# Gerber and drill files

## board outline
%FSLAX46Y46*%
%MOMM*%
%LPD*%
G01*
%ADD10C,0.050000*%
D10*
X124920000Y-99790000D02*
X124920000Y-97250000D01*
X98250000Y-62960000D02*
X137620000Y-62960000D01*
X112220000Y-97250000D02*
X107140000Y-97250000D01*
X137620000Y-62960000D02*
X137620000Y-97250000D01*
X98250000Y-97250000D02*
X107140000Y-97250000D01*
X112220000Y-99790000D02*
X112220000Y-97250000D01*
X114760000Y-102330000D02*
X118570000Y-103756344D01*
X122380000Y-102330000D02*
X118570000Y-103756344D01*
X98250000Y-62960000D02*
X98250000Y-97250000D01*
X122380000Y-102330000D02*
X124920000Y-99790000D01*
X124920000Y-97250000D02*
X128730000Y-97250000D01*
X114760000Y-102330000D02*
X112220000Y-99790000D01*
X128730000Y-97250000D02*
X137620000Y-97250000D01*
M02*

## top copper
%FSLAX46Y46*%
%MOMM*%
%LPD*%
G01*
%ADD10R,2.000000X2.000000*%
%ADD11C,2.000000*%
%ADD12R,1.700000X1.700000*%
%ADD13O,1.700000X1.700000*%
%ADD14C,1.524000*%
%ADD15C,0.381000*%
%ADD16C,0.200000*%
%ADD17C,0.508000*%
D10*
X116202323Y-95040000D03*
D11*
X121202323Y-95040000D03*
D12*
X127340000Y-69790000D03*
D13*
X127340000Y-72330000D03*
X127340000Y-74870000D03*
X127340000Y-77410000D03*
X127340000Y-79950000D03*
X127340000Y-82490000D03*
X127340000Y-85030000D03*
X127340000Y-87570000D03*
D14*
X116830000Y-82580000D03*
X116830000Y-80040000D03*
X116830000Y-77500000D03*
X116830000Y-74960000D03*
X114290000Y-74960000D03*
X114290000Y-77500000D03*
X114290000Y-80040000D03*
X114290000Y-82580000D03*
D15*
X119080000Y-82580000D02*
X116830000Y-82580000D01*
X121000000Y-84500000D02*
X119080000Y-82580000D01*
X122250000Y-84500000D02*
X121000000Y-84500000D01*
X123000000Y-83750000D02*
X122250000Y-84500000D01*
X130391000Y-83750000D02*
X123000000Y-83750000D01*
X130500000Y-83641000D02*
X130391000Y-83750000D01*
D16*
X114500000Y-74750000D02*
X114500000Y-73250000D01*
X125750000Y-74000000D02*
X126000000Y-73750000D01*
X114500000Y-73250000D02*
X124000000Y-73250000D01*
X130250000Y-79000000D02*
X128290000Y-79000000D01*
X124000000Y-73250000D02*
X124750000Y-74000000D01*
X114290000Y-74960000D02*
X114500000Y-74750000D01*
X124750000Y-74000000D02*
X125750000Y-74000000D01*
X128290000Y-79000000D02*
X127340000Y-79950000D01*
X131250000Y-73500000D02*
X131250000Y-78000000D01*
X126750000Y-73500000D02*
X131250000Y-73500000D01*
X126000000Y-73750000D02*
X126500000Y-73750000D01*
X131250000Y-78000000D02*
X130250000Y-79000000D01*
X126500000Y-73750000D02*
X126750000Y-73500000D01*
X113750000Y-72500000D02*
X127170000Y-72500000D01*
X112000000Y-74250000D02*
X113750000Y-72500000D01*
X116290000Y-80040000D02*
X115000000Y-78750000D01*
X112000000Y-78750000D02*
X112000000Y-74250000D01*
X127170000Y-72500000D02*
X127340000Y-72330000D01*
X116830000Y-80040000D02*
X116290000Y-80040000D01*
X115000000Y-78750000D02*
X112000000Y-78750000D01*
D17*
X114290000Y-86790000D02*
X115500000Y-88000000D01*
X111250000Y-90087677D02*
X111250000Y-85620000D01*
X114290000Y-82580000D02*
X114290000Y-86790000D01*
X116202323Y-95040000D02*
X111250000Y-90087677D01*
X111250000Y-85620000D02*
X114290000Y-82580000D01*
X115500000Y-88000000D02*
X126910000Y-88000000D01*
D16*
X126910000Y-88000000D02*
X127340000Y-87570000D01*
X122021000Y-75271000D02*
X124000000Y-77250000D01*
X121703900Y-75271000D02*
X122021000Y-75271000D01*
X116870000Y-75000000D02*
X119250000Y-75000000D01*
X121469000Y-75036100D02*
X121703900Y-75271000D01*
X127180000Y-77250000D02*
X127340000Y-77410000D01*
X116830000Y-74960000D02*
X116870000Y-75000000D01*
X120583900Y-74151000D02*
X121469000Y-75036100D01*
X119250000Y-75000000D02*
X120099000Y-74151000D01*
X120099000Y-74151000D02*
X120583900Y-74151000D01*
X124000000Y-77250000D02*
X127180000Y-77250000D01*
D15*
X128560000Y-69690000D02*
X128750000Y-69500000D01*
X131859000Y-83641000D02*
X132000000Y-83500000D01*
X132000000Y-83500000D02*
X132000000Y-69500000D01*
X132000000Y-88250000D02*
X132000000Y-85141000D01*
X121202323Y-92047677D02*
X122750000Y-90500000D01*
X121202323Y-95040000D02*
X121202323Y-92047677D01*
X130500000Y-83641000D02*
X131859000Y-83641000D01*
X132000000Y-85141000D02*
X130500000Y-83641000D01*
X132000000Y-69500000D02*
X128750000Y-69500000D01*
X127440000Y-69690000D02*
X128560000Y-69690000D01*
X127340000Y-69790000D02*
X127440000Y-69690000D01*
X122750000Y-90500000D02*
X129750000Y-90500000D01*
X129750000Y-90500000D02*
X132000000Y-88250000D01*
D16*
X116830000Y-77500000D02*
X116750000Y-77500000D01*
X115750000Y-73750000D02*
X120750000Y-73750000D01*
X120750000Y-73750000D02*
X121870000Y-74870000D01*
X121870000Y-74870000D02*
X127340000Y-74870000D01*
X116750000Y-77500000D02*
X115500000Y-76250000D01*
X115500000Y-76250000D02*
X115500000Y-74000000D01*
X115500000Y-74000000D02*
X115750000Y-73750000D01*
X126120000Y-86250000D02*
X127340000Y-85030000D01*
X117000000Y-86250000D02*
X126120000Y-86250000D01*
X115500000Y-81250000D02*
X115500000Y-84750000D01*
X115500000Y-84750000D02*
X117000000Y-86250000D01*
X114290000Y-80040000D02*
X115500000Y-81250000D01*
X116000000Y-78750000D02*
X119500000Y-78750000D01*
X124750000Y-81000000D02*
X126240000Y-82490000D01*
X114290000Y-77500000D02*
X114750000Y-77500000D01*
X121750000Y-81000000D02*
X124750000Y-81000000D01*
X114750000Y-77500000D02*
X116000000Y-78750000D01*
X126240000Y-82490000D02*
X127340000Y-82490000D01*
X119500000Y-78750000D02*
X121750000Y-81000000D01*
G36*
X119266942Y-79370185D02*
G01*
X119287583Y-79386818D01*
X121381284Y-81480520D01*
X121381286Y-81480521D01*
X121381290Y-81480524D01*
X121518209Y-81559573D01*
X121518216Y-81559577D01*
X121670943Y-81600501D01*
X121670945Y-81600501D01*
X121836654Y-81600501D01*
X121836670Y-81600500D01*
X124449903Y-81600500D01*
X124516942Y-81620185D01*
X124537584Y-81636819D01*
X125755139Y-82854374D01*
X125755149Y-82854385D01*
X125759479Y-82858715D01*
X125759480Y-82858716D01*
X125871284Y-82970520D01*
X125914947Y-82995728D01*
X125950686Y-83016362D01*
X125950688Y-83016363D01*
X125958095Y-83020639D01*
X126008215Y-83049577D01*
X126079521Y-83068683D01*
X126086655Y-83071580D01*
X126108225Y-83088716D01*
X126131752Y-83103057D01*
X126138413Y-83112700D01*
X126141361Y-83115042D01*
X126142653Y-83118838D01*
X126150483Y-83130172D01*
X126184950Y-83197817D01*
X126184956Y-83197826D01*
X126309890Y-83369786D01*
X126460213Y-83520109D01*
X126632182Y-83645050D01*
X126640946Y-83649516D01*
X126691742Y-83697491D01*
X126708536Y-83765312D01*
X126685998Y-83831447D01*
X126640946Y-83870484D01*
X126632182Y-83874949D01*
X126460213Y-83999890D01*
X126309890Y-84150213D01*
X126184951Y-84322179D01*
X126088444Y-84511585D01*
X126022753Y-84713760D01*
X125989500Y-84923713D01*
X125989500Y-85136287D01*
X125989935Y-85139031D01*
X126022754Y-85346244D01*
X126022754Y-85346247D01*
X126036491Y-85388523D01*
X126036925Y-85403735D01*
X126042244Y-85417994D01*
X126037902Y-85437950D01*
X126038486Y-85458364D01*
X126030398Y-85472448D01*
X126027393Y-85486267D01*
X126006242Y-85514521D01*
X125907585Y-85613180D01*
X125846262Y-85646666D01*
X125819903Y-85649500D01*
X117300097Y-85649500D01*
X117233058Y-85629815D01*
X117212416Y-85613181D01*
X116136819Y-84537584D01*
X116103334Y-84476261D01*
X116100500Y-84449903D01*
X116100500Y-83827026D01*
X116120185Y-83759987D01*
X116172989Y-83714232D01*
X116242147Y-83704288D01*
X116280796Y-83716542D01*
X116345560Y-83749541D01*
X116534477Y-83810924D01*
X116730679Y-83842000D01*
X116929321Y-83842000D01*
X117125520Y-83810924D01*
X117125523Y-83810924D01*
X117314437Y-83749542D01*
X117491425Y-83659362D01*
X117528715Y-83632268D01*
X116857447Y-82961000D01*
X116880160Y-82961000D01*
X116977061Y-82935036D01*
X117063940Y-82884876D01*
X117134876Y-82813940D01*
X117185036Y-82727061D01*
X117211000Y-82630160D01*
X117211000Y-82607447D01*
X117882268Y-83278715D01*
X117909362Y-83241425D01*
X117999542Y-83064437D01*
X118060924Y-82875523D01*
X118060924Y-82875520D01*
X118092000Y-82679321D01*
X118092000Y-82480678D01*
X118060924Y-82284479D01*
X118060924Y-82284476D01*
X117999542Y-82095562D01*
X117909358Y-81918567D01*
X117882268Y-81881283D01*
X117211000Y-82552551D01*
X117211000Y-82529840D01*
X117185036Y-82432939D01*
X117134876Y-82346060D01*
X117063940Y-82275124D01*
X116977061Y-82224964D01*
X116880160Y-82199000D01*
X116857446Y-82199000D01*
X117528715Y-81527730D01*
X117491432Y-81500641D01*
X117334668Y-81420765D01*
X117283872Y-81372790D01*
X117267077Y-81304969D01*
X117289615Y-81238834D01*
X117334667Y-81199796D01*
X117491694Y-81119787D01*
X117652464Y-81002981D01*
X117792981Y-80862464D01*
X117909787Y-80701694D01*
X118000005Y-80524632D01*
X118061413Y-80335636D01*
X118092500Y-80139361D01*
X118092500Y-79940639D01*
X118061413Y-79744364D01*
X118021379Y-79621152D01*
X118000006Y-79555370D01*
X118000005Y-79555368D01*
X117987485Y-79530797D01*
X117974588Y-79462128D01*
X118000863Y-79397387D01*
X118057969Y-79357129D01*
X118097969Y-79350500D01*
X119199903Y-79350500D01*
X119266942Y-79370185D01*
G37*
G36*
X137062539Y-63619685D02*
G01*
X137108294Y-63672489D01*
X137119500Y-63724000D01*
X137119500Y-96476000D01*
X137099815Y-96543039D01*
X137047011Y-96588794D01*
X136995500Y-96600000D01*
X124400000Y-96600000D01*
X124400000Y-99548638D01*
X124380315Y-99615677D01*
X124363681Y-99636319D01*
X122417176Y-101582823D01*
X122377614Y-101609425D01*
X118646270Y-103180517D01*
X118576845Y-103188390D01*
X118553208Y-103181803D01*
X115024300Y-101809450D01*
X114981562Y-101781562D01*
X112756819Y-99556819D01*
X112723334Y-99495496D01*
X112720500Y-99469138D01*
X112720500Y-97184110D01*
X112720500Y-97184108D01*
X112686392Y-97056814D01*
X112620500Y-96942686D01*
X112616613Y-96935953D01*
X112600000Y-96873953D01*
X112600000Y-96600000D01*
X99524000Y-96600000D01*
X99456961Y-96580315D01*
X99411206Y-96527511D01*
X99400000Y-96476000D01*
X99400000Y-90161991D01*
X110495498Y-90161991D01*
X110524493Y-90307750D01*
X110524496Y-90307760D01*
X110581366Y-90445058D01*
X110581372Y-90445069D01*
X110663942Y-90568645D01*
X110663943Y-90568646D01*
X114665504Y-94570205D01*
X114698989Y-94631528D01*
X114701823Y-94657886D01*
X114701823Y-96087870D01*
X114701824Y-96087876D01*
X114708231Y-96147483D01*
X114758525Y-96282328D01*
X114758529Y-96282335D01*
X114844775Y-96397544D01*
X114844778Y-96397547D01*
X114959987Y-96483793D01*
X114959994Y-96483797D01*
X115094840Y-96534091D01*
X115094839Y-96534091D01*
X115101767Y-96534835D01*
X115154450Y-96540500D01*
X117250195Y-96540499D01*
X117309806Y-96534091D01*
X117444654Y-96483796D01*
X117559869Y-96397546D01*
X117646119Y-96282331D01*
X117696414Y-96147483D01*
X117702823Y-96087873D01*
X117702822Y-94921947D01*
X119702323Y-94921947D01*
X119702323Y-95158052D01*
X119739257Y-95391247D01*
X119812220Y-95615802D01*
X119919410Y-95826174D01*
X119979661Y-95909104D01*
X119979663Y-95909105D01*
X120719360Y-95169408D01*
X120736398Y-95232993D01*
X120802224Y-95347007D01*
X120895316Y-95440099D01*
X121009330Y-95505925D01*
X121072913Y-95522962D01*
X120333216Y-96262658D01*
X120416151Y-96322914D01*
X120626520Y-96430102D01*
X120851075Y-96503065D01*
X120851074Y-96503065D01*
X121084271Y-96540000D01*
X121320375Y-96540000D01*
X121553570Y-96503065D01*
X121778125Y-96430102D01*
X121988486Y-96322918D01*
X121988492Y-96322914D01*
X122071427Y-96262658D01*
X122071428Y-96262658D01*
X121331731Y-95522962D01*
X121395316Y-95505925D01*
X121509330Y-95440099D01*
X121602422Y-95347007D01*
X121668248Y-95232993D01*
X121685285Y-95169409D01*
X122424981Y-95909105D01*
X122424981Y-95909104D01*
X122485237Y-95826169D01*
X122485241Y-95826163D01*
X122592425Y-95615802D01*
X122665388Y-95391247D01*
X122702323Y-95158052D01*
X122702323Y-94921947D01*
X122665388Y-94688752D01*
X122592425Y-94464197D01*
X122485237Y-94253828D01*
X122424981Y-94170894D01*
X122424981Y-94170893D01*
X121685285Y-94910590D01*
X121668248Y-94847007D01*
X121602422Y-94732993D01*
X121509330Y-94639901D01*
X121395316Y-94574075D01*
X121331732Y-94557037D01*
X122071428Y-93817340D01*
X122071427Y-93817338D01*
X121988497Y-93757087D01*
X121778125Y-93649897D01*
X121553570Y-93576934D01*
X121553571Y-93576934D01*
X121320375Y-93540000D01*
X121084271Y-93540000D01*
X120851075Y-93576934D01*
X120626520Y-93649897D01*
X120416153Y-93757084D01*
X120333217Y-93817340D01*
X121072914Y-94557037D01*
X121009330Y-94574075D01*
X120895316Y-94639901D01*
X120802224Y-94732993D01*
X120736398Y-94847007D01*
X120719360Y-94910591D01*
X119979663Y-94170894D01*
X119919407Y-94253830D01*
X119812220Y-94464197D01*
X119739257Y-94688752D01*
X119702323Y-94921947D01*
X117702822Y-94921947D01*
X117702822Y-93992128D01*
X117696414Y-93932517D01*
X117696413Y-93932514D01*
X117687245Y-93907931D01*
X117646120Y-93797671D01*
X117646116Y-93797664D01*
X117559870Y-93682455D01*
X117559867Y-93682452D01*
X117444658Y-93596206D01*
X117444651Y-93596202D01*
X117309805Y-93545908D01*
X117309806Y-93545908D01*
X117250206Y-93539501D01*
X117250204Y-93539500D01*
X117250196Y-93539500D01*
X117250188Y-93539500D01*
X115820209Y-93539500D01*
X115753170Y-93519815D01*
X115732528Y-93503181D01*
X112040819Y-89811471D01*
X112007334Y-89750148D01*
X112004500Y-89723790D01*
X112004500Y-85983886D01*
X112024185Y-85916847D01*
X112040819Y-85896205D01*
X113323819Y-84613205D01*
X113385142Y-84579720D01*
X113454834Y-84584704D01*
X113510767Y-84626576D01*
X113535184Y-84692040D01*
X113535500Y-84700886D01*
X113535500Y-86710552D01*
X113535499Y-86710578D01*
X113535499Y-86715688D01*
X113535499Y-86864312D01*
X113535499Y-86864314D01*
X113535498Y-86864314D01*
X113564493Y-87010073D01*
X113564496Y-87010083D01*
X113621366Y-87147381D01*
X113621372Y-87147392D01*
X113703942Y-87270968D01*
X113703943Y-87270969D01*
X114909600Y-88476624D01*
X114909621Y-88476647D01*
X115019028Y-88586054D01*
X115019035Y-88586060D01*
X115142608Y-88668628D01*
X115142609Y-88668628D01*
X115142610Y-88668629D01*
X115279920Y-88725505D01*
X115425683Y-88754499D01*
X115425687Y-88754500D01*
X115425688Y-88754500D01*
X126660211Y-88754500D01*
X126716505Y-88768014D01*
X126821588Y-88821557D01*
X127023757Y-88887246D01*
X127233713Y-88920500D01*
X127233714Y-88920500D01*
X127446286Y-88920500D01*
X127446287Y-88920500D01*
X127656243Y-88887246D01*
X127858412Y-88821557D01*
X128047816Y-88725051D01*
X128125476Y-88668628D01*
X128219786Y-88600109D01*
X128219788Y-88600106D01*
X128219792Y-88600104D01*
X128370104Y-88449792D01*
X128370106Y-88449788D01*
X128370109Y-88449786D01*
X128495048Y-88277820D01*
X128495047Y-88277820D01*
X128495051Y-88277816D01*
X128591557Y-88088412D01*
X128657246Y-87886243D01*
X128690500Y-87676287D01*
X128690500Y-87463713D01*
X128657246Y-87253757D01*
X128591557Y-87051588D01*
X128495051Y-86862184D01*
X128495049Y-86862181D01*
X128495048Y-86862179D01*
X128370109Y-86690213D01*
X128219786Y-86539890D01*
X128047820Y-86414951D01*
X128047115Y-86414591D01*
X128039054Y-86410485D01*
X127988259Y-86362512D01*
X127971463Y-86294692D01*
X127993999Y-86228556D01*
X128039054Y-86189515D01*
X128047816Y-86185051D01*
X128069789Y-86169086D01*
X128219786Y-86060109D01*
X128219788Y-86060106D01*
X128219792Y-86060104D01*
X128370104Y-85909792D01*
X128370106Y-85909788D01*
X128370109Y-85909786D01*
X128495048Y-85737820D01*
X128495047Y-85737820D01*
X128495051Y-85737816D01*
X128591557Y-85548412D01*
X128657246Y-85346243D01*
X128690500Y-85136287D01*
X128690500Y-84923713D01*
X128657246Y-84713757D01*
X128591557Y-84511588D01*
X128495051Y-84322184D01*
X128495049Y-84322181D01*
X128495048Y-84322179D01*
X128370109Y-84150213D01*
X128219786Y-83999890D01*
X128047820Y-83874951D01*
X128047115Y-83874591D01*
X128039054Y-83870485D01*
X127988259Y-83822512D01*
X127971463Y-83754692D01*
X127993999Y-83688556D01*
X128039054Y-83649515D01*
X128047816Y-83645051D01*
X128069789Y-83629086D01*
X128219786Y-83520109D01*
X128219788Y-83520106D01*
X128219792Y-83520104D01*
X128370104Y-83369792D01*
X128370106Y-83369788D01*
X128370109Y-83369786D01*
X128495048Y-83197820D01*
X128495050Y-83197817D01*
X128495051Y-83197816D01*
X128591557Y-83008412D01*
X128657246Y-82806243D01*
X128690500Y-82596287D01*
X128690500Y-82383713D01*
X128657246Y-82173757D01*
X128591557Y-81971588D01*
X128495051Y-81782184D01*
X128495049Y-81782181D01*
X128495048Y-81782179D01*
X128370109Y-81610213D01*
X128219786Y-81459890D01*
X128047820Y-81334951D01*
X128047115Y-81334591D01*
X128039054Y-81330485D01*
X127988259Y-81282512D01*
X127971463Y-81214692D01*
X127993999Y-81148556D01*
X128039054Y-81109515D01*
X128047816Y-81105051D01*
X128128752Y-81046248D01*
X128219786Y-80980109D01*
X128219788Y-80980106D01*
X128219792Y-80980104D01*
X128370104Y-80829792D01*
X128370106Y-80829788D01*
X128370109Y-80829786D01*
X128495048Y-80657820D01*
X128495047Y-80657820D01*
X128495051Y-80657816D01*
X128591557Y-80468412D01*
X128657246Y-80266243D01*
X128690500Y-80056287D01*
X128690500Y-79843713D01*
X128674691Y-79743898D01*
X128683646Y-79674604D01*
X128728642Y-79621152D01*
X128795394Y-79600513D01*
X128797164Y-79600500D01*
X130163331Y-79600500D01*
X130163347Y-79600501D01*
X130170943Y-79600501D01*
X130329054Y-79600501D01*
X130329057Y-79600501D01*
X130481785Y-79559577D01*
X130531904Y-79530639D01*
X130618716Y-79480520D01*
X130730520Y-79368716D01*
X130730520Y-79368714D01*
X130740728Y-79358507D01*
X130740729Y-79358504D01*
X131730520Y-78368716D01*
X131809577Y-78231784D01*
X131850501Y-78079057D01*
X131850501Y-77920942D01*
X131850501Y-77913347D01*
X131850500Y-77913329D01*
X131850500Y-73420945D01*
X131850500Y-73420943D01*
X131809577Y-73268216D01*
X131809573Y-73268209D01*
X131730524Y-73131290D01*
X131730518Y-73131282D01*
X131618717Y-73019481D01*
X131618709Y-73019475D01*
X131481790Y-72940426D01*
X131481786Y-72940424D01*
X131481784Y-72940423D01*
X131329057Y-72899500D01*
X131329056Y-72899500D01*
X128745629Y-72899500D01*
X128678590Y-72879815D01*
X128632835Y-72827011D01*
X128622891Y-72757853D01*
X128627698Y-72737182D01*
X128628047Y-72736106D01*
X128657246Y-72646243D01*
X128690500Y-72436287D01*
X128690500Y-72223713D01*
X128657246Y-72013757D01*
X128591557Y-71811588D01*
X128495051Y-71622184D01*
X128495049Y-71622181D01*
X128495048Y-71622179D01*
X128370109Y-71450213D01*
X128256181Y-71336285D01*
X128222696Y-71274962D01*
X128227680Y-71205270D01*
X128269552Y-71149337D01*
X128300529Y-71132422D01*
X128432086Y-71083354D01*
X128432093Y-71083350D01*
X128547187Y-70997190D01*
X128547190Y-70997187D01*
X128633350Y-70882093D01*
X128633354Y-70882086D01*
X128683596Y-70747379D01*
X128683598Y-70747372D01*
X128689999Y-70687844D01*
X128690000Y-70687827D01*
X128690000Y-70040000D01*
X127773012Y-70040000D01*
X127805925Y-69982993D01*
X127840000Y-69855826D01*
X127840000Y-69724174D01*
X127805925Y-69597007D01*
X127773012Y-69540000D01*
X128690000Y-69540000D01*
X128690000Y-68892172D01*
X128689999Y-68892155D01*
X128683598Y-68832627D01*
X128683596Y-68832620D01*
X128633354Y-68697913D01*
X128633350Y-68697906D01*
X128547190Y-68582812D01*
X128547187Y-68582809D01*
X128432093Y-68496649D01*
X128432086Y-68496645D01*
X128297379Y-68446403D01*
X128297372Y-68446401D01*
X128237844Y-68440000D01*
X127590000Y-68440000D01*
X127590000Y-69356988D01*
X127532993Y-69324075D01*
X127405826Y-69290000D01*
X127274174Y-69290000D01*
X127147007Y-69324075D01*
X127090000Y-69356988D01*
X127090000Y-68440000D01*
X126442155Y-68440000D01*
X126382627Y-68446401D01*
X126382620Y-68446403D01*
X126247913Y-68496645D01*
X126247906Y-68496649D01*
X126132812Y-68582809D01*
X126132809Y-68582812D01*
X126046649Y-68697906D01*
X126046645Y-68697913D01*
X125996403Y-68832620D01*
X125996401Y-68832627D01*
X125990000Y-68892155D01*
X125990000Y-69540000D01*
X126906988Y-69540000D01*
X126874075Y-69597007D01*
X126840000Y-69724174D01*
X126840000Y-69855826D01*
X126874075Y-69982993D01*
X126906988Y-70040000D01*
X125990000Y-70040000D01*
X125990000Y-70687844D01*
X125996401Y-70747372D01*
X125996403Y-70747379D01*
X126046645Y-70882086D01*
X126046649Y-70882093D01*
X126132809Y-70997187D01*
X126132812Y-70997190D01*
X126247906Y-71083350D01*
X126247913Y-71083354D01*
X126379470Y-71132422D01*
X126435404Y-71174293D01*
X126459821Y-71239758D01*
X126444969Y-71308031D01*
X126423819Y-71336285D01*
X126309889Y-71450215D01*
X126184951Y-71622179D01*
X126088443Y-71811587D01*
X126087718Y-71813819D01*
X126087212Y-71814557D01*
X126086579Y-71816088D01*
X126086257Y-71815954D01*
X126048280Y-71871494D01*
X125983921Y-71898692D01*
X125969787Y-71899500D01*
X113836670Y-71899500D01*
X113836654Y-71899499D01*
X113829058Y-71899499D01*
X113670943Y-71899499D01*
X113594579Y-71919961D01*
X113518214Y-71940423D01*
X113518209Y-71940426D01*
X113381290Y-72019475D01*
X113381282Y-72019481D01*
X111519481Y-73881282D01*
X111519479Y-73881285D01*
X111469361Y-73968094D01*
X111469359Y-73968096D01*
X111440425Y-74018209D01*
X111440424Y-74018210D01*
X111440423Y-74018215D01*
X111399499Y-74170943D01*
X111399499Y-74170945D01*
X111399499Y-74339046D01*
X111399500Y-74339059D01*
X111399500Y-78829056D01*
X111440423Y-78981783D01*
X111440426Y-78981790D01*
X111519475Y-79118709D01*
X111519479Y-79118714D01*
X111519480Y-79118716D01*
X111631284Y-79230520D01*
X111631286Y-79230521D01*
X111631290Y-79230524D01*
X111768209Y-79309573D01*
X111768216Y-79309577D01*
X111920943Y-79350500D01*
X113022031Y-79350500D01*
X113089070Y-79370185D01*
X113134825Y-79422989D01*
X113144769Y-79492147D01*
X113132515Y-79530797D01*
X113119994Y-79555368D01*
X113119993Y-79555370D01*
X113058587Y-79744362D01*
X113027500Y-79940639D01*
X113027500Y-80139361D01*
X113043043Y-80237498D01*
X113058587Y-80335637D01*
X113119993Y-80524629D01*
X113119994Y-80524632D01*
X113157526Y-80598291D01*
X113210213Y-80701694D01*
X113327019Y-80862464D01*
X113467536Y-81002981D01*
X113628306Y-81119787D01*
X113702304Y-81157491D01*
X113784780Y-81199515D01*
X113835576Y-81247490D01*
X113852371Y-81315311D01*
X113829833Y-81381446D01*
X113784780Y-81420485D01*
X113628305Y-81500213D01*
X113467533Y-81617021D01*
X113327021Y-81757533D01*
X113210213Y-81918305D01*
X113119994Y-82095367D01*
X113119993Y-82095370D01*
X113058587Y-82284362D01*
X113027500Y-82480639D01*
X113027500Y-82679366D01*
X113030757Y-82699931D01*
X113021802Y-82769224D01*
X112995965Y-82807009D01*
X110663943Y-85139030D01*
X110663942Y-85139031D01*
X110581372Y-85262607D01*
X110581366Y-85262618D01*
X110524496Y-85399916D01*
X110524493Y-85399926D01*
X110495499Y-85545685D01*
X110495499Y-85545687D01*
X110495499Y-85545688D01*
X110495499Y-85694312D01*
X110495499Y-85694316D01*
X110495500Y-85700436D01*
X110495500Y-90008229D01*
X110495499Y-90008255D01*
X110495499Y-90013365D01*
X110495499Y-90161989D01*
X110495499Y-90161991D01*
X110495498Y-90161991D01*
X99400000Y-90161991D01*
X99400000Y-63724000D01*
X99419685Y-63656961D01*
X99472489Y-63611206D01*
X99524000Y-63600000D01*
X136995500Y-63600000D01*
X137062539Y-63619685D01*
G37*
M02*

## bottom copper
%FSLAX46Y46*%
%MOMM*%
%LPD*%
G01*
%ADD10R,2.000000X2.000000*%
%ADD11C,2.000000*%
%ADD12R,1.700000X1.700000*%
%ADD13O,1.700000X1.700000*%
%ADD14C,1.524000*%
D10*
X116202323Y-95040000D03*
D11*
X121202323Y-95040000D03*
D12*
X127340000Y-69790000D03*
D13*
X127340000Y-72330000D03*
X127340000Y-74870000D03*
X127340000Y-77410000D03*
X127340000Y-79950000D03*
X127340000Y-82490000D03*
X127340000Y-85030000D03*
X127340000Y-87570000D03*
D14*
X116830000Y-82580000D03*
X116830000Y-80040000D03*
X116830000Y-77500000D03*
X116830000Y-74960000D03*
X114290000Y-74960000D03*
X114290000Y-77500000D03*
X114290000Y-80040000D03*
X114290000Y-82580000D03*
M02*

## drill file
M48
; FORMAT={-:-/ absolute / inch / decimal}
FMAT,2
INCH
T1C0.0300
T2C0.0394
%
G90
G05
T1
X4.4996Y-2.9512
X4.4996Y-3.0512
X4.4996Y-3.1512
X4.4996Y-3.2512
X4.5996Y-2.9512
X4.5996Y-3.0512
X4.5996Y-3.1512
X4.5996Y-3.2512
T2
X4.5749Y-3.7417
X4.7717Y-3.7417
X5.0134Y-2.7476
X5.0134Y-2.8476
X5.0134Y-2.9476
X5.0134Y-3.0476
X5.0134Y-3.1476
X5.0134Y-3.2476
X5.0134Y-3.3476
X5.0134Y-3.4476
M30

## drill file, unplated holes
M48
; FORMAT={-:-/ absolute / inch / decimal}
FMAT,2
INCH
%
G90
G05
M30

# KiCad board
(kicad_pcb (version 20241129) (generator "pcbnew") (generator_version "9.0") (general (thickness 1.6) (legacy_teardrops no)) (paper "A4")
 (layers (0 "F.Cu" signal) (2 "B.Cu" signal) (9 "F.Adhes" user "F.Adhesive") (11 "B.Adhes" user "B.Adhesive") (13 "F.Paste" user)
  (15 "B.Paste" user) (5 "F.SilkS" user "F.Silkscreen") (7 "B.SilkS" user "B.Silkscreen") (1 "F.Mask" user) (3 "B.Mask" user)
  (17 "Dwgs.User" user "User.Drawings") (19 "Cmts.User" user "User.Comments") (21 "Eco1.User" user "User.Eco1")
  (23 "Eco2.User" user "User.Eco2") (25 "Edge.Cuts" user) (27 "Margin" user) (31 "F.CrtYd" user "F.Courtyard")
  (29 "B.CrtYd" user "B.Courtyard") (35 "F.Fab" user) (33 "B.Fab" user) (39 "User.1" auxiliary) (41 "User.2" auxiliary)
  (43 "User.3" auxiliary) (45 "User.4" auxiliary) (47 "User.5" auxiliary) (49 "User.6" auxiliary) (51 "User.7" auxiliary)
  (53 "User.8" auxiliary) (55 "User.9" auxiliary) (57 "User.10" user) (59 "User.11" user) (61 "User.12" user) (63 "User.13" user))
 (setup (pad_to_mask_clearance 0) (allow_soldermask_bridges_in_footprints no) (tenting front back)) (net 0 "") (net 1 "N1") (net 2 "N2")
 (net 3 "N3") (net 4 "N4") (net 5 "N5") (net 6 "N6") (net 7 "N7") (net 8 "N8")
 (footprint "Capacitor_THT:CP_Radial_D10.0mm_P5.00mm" (layer "F.Cu") (at 116.202323 95.04)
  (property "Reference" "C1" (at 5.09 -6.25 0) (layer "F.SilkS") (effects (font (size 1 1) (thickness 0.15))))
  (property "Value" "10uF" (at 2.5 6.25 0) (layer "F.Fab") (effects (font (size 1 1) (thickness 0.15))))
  (pad "1" thru_hole rect (at 0 0) (size 2 2) (drill 1) (layers "*.Cu" "*.Mask") (remove_unused_layers no) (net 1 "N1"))
  (pad "2" thru_hole circle (at 5 0) (size 2 2) (drill 1) (layers "*.Cu" "*.Mask") (remove_unused_layers no) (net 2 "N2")))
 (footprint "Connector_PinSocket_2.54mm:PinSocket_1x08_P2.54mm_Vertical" (layer "F.Cu") (at 127.34 69.79)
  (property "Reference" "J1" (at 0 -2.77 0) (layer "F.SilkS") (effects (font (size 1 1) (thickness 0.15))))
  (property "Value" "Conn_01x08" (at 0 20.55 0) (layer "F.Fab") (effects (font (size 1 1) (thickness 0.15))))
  (pad "1" thru_hole rect (at 0 0) (size 1.7 1.7) (drill 1) (layers "*.Cu" "*.Mask") (remove_unused_layers no) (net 2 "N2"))
  (pad "2" thru_hole oval (at 0 2.54) (size 1.7 1.7) (drill 1) (layers "*.Cu" "*.Mask") (remove_unused_layers no) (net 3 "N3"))
  (pad "3" thru_hole oval (at 0 5.08) (size 1.7 1.7) (drill 1) (layers "*.Cu" "*.Mask") (remove_unused_layers no) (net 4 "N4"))
  (pad "4" thru_hole oval (at 0 7.62) (size 1.7 1.7) (drill 1) (layers "*.Cu" "*.Mask") (remove_unused_layers no) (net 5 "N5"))
  (pad "5" thru_hole oval (at 0 10.16) (size 1.7 1.7) (drill 1) (layers "*.Cu" "*.Mask") (remove_unused_layers no) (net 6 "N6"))
  (pad "6" thru_hole oval (at 0 12.7) (size 1.7 1.7) (drill 1) (layers "*.Cu" "*.Mask") (remove_unused_layers no) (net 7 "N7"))
  (pad "7" thru_hole oval (at 0 15.24) (size 1.7 1.7) (drill 1) (layers "*.Cu" "*.Mask") (remove_unused_layers no) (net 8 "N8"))
  (pad "8" thru_hole oval (at 0 17.78) (size 1.7 1.7) (drill 1) (layers "*.Cu" "*.Mask") (remove_unused_layers no) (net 1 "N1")))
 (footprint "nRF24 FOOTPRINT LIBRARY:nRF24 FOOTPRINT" (layer "F.Cu") (at 111.75 77.5)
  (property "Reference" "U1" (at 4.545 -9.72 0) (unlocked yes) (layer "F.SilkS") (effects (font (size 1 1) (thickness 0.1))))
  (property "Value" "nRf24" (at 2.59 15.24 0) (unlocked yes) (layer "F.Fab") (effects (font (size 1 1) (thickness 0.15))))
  (pad "0" thru_hole circle (at 5.08 5.08) (size 1.524 1.524) (drill 0.762) (layers "*.Cu" "*.Mask") (remove_unused_layers no) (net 2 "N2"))
  (pad "1" thru_hole circle (at 5.08 2.54) (size 1.524 1.524) (drill 0.762) (layers "*.Cu" "*.Mask") (remove_unused_layers no) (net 3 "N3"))
  (pad "2" thru_hole circle (at 5.08 0) (size 1.524 1.524) (drill 0.762) (layers "*.Cu" "*.Mask") (remove_unused_layers no) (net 4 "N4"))
  (pad "3" thru_hole circle (at 5.08 -2.54) (size 1.524 1.524) (drill 0.762) (layers "*.Cu" "*.Mask") (remove_unused_layers no) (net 5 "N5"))
  (pad "4" thru_hole circle (at 2.54 -2.54) (size 1.524 1.524) (drill 0.762) (layers "*.Cu" "*.Mask") (remove_unused_layers no) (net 6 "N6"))
  (pad "5" thru_hole circle (at 2.54 0) (size 1.524 1.524) (drill 0.762) (layers "*.Cu" "*.Mask") (remove_unused_layers no) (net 7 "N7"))
  (pad "6" thru_hole circle (at 2.54 2.54) (size 1.524 1.524) (drill 0.762) (layers "*.Cu" "*.Mask") (remove_unused_layers no) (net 8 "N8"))
  (pad "7" thru_hole circle (at 2.54 5.08) (size 1.524 1.524) (drill 0.762) (layers "*.Cu" "*.Mask") (remove_unused_layers no) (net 1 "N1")))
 (gr_line (start 124.92 99.79) (end 124.92 97.25) (stroke (width 0.05) (type default)) (layer "Edge.Cuts"))
 (gr_line (start 98.25 62.96) (end 137.62 62.96) (stroke (width 0.05) (type default)) (layer "Edge.Cuts"))
 (gr_line (start 112.22 97.25) (end 107.14 97.25) (stroke (width 0.05) (type default)) (layer "Edge.Cuts"))
 (gr_line (start 137.62 62.96) (end 137.62 97.25) (stroke (width 0.05) (type default)) (layer "Edge.Cuts"))
 (gr_line (start 98.25 97.25) (end 107.14 97.25) (stroke (width 0.05) (type default)) (layer "Edge.Cuts"))
 (gr_line (start 112.22 99.79) (end 112.22 97.25) (stroke (width 0.05) (type default)) (layer "Edge.Cuts"))
 (gr_line (start 114.76 102.33) (end 118.57 103.756344) (stroke (width 0.05) (type default)) (layer "Edge.Cuts"))
 (gr_line (start 122.38 102.33) (end 118.57 103.756344) (stroke (width 0.05) (type default)) (layer "Edge.Cuts"))
 (gr_line (start 98.25 62.96) (end 98.25 97.25) (stroke (width 0.05) (type default)) (layer "Edge.Cuts"))
 (gr_line (start 122.38 102.33) (end 124.92 99.79) (stroke (width 0.05) (type default)) (layer "Edge.Cuts"))
 (gr_line (start 124.92 97.25) (end 128.73 97.25) (stroke (width 0.05) (type default)) (layer "Edge.Cuts"))
 (gr_line (start 114.76 102.33) (end 112.22 99.79) (stroke (width 0.05) (type default)) (layer "Edge.Cuts"))
 (gr_line (start 128.73 97.25) (end 137.62 97.25) (stroke (width 0.05) (type default)) (layer "Edge.Cuts"))
 (segment (start 114.5 74.75) (end 114.5 73.25) (width 0.2) (layer "F.Cu") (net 6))
 (segment (start 125.75 74) (end 126 73.75) (width 0.2) (layer "F.Cu") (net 6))
 (segment (start 114.5 73.25) (end 124 73.25) (width 0.2) (layer "F.Cu") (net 6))
 (segment (start 130.25 79) (end 128.29 79) (width 0.2) (layer "F.Cu") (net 6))
 (segment (start 124 73.25) (end 124.75 74) (width 0.2) (layer "F.Cu") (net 6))
 (segment (start 114.29 74.96) (end 114.5 74.75) (width 0.2) (layer "F.Cu") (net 6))
 (segment (start 124.75 74) (end 125.75 74) (width 0.2) (layer "F.Cu") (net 6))
 (segment (start 128.29 79) (end 127.34 79.95) (width 0.2) (layer "F.Cu") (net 6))
 (segment (start 131.25 73.5) (end 131.25 78) (width 0.2) (layer "F.Cu") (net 6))
 (segment (start 126.75 73.5) (end 131.25 73.5) (width 0.2) (layer "F.Cu") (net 6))
 (segment (start 126 73.75) (end 126.5 73.75) (width 0.2) (layer "F.Cu") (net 6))
 (segment (start 131.25 78) (end 130.25 79) (width 0.2) (layer "F.Cu") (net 6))
 (segment (start 126.5 73.75) (end 126.75 73.5) (width 0.2) (layer "F.Cu") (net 6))
 (segment (start 113.75 72.5) (end 127.17 72.5) (width 0.2) (layer "F.Cu") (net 3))
 (segment (start 112 74.25) (end 113.75 72.5) (width 0.2) (layer "F.Cu") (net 3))
 (segment (start 116.29 80.04) (end 115 78.75) (width 0.2) (layer "F.Cu") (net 3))
 (segment (start 112 78.75) (end 112 74.25) (width 0.2) (layer "F.Cu") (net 3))
 (segment (start 127.17 72.5) (end 127.34 72.33) (width 0.2) (layer "F.Cu") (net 3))
 (segment (start 116.83 80.04) (end 116.29 80.04) (width 0.2) (layer "F.Cu") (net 3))
 (segment (start 115 78.75) (end 112 78.75) (width 0.2) (layer "F.Cu") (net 3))
 (segment (start 114.29 86.79) (end 115.5 88) (width 0.508) (layer "F.Cu") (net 1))
 (segment (start 111.25 90.087677) (end 111.25 85.62) (width 0.508) (layer "F.Cu") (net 1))
 (segment (start 114.29 82.58) (end 114.29 86.79) (width 0.508) (layer "F.Cu") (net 1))
 (segment (start 116.202323 95.04) (end 111.25 90.087677) (width 0.508) (layer "F.Cu") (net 1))
 (segment (start 111.25 85.62) (end 114.29 82.58) (width 0.508) (layer "F.Cu") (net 1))
 (segment (start 115.5 88) (end 126.91 88) (width 0.508) (layer "F.Cu") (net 1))
 (segment (start 126.91 88) (end 127.34 87.57) (width 0.2) (layer "F.Cu") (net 1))
 (segment (start 122.021 75.271) (end 124 77.25) (width 0.2) (layer "F.Cu") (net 5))
 (segment (start 121.7039 75.271) (end 122.021 75.271) (width 0.2) (layer "F.Cu") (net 5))
 (segment (start 116.87 75) (end 119.25 75) (width 0.2) (layer "F.Cu") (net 5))
 (segment (start 121.469 75.0361) (end 121.7039 75.271) (width 0.2) (layer "F.Cu") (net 5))
 (segment (start 127.18 77.25) (end 127.34 77.41) (width 0.2) (layer "F.Cu") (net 5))
 (segment (start 116.83 74.96) (end 116.87 75) (width 0.2) (layer "F.Cu") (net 5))
 (segment (start 120.5839 74.151) (end 121.469 75.0361) (width 0.2) (layer "F.Cu") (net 5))
 (segment (start 119.25 75) (end 120.099 74.151) (width 0.2) (layer "F.Cu") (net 5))
 (segment (start 120.099 74.151) (end 120.5839 74.151) (width 0.2) (layer "F.Cu") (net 5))
 (segment (start 124 77.25) (end 127.18 77.25) (width 0.2) (layer "F.Cu") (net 5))
 (segment (start 128.56 69.69) (end 128.75 69.5) (width 0.381) (layer "F.Cu") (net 2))
 (segment (start 131.859 83.641) (end 132 83.5) (width 0.381) (layer "F.Cu") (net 2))
 (segment (start 132 83.5) (end 132 69.5) (width 0.381) (layer "F.Cu") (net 2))
 (segment (start 132 88.25) (end 132 85.141) (width 0.381) (layer "F.Cu") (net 2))
 (segment (start 121.202323 92.047677) (end 122.75 90.5) (width 0.381) (layer "F.Cu") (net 2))
 (segment (start 123 83.75) (end 122.25 84.5) (width 0.381) (layer "F.Cu") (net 2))
 (segment (start 121.202323 95.04) (end 121.202323 92.047677) (width 0.381) (layer "F.Cu") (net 2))
 (segment (start 130.5 83.641) (end 131.859 83.641) (width 0.381) (layer "F.Cu") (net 2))
 (segment (start 130.391 83.75) (end 123 83.75) (width 0.381) (layer "F.Cu") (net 2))
 (segment (start 122.25 84.5) (end 121 84.5) (width 0.381) (layer "F.Cu") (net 2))
 (segment (start 132 85.141) (end 130.5 83.641) (width 0.381) (layer "F.Cu") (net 2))
 (segment (start 121 84.5) (end 119.08 82.58) (width 0.381) (layer "F.Cu") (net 2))
 (segment (start 132 69.5) (end 128.75 69.5) (width 0.381) (layer "F.Cu") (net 2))
 (segment (start 119.08 82.58) (end 116.83 82.58) (width 0.381) (layer "F.Cu") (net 2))
 (segment (start 127.44 69.69) (end 128.56 69.69) (width 0.381) (layer "F.Cu") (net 2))
 (segment (start 130.5 83.641) (end 130.391 83.75) (width 0.381) (layer "F.Cu") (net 2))
 (segment (start 127.34 69.79) (end 127.44 69.69) (width 0.381) (layer "F.Cu") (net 2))
 (segment (start 122.75 90.5) (end 129.75 90.5) (width 0.381) (layer "F.Cu") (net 2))
 (segment (start 129.75 90.5) (end 132 88.25) (width 0.381) (layer "F.Cu") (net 2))
 (segment (start 116.83 77.5) (end 116.75 77.5) (width 0.2) (layer "F.Cu") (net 4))
 (segment (start 115.75 73.75) (end 120.75 73.75) (width 0.2) (layer "F.Cu") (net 4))
 (segment (start 120.75 73.75) (end 121.87 74.87) (width 0.2) (layer "F.Cu") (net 4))
 (segment (start 121.87 74.87) (end 127.34 74.87) (width 0.2) (layer "F.Cu") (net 4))
 (segment (start 116.75 77.5) (end 115.5 76.25) (width 0.2) (layer "F.Cu") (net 4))
 (segment (start 115.5 76.25) (end 115.5 74) (width 0.2) (layer "F.Cu") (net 4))
 (segment (start 115.5 74) (end 115.75 73.75) (width 0.2) (layer "F.Cu") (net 4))
 (segment (start 126.12 86.25) (end 127.34 85.03) (width 0.2) (layer "F.Cu") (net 8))
 (segment (start 117 86.25) (end 126.12 86.25) (width 0.2) (layer "F.Cu") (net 8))
 (segment (start 115.5 81.25) (end 115.5 84.75) (width 0.2) (layer "F.Cu") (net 8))
 (segment (start 115.5 84.75) (end 117 86.25) (width 0.2) (layer "F.Cu") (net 8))
 (segment (start 114.29 80.04) (end 115.5 81.25) (width 0.2) (layer "F.Cu") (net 8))
 (segment (start 116 78.75) (end 119.5 78.75) (width 0.2) (layer "F.Cu") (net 7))
 (segment (start 124.75 81) (end 126.24 82.49) (width 0.2) (layer "F.Cu") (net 7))
 (segment (start 114.29 77.5) (end 114.75 77.5) (width 0.2) (layer "F.Cu") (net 7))
 (segment (start 121.75 81) (end 124.75 81) (width 0.2) (layer "F.Cu") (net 7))
 (segment (start 114.75 77.5) (end 116 78.75) (width 0.2) (layer "F.Cu") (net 7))
 (segment (start 126.24 82.49) (end 127.34 82.49) (width 0.2) (layer "F.Cu") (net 7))
 (segment (start 119.5 78.75) (end 121.75 81) (width 0.2) (layer "F.Cu") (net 7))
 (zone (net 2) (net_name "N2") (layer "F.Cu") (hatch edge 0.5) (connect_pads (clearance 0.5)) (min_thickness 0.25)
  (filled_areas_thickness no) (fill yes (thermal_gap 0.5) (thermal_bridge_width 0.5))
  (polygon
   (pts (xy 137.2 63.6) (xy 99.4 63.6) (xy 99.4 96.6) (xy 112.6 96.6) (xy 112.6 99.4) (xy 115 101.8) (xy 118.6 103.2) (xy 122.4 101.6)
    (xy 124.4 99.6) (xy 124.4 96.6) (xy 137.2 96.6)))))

